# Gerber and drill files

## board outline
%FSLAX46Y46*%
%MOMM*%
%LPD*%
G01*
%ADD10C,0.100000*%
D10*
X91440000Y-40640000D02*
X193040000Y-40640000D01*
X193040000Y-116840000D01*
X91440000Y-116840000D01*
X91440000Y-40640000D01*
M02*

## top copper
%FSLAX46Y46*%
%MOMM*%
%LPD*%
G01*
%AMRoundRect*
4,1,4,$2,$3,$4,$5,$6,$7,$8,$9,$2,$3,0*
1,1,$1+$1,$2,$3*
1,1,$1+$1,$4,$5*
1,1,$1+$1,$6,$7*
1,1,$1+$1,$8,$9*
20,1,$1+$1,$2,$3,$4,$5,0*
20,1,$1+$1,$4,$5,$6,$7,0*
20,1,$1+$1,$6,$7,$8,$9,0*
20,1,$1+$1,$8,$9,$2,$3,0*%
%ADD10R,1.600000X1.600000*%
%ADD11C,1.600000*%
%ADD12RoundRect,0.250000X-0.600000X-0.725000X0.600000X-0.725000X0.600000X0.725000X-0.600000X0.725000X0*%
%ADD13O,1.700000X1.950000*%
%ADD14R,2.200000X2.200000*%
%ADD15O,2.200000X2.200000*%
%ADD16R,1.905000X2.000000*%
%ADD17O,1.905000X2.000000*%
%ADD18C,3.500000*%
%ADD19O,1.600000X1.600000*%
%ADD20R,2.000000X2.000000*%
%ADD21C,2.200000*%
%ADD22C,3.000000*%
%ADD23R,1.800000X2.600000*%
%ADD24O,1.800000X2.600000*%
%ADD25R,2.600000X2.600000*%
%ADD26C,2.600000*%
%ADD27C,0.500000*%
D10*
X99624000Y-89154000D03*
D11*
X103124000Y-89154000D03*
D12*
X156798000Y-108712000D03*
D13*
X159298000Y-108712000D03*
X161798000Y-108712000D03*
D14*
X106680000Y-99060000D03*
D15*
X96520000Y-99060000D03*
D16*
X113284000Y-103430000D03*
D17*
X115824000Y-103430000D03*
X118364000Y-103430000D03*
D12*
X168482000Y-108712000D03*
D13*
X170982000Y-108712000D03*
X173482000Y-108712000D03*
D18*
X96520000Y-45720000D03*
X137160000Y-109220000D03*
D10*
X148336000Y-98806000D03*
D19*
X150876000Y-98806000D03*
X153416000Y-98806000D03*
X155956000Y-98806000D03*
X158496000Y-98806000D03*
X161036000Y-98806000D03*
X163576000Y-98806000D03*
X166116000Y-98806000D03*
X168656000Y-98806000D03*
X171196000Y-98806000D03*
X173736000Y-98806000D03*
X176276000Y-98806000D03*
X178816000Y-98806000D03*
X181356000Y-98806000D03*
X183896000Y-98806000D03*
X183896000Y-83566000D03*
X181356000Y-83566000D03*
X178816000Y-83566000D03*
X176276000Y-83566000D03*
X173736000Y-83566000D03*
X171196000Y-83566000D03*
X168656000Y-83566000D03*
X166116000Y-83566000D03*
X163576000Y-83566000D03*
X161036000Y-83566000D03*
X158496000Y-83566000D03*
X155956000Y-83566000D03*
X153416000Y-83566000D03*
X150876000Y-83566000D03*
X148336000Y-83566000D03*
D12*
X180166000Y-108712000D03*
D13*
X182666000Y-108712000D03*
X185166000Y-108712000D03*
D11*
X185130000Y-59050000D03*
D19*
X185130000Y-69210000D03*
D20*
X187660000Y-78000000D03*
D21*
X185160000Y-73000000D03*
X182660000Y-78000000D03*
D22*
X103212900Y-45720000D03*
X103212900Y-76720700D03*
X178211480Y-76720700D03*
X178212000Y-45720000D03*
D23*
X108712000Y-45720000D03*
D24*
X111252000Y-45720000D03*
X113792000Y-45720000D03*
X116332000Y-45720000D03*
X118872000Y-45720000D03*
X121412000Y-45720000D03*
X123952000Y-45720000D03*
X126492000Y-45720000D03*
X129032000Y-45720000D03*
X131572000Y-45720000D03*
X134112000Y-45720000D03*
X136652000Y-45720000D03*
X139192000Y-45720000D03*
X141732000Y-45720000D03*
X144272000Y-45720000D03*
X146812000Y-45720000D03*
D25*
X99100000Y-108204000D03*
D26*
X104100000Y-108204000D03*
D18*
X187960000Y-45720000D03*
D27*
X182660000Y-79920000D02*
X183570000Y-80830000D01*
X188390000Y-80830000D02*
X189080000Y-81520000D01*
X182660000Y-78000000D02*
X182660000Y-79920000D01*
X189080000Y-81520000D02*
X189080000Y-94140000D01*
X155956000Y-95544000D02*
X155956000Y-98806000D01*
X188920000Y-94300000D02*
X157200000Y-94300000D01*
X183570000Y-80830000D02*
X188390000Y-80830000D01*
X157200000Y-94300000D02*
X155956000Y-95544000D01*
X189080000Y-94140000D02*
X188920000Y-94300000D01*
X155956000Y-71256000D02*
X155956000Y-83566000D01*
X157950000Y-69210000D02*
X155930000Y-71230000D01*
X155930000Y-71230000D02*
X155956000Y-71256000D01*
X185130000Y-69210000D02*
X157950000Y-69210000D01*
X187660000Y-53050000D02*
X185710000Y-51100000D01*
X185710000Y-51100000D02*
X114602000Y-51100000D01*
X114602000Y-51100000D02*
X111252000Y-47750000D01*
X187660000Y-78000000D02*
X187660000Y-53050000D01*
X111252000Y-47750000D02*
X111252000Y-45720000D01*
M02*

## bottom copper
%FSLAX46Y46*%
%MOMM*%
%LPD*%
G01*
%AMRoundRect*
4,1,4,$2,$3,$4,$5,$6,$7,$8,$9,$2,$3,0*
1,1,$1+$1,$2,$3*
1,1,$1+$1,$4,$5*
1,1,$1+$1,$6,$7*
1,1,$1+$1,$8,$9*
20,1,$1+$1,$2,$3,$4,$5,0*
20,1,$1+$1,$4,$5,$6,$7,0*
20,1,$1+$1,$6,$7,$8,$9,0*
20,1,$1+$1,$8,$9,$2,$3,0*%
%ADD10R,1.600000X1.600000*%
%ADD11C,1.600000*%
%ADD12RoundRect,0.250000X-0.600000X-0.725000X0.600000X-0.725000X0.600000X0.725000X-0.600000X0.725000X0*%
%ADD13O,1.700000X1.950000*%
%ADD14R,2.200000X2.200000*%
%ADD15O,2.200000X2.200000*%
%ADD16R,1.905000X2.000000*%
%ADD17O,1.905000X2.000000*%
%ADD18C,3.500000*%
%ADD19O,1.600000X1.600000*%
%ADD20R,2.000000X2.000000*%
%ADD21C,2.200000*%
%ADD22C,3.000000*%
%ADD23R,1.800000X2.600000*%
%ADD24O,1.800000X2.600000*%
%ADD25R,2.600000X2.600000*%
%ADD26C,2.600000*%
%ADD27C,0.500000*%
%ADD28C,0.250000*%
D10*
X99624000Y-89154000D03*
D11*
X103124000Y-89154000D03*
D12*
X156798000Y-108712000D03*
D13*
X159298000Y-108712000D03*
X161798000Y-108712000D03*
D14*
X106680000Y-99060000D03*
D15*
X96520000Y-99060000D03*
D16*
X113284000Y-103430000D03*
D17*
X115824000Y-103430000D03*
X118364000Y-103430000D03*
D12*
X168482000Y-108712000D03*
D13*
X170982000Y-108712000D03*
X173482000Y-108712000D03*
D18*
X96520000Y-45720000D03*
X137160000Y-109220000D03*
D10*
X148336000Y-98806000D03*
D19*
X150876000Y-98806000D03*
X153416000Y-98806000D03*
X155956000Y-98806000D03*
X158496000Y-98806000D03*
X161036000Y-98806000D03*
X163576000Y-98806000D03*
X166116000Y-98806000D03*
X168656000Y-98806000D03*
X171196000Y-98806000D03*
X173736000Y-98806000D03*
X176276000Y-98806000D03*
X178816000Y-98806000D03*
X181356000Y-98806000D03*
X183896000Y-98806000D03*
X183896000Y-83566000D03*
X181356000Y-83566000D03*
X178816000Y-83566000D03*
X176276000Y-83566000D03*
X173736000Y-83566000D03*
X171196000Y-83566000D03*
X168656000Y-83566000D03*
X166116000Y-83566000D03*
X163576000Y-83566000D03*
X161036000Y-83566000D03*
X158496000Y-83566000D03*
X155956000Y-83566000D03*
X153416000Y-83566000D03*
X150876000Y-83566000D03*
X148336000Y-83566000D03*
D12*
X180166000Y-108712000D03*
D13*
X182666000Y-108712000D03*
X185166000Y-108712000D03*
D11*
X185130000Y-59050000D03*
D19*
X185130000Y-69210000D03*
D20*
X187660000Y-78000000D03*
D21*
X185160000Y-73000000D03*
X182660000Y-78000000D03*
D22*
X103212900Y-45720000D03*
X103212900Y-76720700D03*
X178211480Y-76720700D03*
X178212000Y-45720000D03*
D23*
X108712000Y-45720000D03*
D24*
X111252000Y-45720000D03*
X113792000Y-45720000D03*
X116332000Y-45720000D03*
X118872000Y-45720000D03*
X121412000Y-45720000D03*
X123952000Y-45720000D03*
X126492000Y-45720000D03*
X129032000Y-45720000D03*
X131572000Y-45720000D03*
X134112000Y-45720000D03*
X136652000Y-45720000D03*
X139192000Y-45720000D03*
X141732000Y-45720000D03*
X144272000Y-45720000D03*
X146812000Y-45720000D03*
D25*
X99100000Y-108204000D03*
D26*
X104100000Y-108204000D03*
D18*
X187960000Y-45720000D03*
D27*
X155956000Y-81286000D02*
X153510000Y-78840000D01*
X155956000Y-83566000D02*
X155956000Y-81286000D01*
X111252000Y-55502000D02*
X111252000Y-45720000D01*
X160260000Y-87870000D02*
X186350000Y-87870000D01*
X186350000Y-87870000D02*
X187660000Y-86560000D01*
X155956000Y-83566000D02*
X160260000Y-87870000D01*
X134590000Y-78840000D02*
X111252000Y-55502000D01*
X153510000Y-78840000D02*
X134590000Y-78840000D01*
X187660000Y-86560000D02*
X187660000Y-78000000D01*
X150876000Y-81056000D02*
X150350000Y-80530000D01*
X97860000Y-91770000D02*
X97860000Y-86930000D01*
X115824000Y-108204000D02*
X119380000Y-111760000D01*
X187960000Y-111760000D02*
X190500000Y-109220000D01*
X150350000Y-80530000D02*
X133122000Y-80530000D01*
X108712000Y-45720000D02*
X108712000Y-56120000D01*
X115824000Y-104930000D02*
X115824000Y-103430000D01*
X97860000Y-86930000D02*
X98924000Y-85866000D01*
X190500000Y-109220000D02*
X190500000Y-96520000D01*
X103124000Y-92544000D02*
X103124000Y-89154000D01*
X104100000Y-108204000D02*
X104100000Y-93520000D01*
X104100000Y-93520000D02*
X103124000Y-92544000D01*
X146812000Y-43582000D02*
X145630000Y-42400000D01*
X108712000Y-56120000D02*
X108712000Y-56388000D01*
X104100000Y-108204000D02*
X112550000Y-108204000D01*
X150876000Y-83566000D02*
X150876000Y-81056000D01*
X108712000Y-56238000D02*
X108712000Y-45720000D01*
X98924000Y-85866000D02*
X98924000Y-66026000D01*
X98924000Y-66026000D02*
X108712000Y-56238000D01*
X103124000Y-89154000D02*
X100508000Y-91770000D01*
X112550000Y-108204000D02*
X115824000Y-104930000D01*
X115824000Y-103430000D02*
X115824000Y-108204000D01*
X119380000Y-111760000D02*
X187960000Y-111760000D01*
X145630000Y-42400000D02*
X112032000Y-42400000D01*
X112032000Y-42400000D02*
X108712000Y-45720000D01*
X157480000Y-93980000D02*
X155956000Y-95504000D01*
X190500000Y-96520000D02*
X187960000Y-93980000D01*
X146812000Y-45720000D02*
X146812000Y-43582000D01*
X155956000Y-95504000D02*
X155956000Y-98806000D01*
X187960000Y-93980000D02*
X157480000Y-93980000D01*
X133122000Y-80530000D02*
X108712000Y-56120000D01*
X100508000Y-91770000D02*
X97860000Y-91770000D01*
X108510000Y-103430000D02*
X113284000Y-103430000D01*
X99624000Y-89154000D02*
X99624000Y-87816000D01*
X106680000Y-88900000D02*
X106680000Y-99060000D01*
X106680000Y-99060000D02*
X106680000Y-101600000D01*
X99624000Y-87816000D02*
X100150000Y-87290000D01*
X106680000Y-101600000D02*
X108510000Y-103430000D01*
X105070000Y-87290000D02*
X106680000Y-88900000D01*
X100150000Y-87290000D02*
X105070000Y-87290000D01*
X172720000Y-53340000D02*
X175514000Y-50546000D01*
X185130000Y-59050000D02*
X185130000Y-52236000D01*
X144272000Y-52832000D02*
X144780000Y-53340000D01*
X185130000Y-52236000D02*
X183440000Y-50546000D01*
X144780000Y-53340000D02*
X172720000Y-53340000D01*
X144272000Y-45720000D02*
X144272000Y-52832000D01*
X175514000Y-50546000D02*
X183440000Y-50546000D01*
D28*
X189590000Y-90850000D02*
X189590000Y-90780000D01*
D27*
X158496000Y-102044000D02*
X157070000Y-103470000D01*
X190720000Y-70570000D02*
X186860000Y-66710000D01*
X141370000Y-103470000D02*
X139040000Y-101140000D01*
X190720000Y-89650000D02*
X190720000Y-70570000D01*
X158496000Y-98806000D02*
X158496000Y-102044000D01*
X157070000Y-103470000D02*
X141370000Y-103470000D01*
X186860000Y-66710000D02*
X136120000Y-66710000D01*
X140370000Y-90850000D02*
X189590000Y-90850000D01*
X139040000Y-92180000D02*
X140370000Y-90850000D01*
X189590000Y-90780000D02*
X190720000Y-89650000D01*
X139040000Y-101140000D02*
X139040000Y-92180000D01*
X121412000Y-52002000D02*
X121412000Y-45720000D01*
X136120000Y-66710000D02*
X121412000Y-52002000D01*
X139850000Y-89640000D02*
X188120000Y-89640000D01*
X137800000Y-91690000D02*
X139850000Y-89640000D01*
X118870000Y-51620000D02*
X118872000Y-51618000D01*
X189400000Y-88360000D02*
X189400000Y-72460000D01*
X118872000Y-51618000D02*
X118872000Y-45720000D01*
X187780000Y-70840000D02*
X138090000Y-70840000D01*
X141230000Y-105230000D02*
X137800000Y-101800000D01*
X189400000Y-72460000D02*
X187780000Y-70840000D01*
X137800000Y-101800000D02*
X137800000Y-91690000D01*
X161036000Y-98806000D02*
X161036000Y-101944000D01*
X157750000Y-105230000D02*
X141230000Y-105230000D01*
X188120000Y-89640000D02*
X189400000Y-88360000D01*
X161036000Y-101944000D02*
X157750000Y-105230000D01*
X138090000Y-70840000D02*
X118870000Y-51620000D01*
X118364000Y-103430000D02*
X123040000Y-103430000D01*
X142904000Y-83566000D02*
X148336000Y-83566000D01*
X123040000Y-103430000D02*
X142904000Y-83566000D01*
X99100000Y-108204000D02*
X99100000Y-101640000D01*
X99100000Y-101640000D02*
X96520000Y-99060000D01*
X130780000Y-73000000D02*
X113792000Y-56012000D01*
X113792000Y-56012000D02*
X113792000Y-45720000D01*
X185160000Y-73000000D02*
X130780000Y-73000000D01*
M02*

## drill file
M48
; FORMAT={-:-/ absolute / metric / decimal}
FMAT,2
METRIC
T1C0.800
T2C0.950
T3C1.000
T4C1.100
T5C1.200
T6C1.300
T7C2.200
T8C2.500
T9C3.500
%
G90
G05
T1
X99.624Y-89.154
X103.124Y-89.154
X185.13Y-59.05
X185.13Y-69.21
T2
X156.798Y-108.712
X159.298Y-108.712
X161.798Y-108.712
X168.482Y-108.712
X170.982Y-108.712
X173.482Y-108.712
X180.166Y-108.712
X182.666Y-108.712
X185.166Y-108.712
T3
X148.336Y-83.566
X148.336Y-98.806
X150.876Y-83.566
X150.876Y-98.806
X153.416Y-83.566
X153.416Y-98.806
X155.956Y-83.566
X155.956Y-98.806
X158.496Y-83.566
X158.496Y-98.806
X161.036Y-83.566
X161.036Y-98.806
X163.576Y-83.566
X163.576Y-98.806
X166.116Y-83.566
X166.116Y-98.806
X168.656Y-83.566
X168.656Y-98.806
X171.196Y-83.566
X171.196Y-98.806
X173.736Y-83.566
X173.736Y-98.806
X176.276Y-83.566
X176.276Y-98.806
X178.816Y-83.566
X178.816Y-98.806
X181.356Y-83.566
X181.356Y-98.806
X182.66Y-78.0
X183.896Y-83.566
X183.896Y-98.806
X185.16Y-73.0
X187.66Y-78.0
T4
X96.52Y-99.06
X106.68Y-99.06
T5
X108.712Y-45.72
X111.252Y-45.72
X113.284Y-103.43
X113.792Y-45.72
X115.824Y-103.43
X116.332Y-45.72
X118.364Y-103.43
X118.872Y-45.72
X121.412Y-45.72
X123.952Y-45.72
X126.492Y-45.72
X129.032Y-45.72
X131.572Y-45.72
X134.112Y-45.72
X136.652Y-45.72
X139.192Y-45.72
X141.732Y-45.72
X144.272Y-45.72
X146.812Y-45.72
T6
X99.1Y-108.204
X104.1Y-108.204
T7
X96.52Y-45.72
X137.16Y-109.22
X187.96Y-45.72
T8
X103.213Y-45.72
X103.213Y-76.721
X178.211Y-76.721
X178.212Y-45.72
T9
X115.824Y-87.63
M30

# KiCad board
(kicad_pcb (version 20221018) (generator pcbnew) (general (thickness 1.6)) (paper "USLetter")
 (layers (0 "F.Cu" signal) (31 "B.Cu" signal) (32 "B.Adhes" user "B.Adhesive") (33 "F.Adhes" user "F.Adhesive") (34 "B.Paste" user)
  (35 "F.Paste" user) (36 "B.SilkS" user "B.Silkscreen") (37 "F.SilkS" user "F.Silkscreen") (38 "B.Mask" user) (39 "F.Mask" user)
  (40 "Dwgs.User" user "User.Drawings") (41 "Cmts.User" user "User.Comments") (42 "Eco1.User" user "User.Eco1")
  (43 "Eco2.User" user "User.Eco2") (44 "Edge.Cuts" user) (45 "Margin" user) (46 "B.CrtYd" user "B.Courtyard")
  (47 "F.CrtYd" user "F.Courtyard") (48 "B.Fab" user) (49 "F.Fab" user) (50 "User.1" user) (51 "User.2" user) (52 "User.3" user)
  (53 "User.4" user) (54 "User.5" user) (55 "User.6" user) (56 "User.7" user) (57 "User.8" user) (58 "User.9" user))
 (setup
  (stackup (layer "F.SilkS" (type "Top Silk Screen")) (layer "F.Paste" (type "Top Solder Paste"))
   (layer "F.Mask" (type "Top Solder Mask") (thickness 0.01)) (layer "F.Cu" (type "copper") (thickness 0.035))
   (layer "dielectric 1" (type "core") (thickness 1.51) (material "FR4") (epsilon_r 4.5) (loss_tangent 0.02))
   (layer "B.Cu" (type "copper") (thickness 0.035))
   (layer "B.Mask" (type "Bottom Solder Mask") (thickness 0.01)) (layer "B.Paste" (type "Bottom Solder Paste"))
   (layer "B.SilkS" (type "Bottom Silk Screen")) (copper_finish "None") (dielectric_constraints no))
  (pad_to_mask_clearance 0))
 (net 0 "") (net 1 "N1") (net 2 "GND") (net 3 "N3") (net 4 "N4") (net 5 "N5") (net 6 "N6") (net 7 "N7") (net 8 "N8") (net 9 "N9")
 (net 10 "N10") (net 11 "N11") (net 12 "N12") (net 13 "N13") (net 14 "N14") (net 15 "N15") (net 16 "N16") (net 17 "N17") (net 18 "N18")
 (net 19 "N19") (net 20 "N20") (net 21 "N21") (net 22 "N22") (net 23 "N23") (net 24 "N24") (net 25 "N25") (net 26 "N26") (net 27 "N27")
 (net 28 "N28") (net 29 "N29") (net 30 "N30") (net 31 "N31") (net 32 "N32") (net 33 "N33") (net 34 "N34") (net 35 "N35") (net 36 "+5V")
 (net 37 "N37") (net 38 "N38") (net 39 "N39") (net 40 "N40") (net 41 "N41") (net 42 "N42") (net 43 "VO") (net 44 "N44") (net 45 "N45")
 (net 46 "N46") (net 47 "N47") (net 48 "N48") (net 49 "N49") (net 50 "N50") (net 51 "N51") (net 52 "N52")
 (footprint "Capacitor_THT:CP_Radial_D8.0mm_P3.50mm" (layer "F.Cu") (at 99.624 89.154)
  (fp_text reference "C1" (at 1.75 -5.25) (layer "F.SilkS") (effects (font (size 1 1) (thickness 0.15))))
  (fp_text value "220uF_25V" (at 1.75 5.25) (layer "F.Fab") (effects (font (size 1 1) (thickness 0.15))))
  (pad "1" thru_hole rect (at 0 0) (size 1.6 1.6) (drill 0.8) (layers "*.Cu" "*.Mask") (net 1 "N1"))
  (pad "2" thru_hole circle (at 3.5 0) (size 1.6 1.6) (drill 0.8) (layers "*.Cu" "*.Mask") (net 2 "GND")))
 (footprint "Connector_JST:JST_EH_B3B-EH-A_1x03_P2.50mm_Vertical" (layer "F.Cu") (at 156.798 108.712)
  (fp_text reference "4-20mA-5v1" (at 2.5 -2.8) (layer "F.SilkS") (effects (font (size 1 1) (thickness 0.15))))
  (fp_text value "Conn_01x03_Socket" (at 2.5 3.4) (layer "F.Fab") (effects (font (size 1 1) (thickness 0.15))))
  (pad "1" thru_hole roundrect (at 0 0) (size 1.7 1.95) (drill 0.95) (layers "*.Cu" "*.Mask") (roundrect_rratio 0.147059) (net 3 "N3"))
  (pad "2" thru_hole oval (at 2.5 0) (size 1.7 1.95) (drill 0.95) (layers "*.Cu" "*.Mask") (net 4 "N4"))
  (pad "3" thru_hole oval (at 5 0) (size 1.7 1.95) (drill 0.95) (layers "*.Cu" "*.Mask") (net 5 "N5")))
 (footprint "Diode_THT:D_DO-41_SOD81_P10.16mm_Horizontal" (layer "F.Cu") (at 106.68 99.06 180)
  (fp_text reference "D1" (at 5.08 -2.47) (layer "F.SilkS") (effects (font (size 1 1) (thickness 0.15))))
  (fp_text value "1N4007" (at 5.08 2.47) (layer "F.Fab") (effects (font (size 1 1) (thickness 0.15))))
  (pad "1" thru_hole rect (at 0 0 180) (size 2.2 2.2) (drill 1.1) (layers "*.Cu" "*.Mask") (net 1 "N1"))
  (pad "2" thru_hole oval (at 10.16 0 180) (size 2.2 2.2) (drill 1.1) (layers "*.Cu" "*.Mask") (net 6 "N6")))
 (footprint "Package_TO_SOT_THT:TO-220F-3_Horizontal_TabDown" (layer "F.Cu") (at 113.284 103.43)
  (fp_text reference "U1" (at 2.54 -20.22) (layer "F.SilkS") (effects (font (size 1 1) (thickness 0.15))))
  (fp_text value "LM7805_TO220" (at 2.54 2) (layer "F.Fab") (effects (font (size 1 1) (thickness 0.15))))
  (pad "" np_thru_hole oval (at 2.54 -15.8) (size 3.5 3.5) (drill 3.5) (layers "*.Cu" "*.Mask"))
  (pad "1" thru_hole rect (at 0 0) (size 1.905 2) (drill 1.2) (layers "*.Cu" "*.Mask") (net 1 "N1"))
  (pad "2" thru_hole oval (at 2.54 0) (size 1.905 2) (drill 1.2) (layers "*.Cu" "*.Mask") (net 2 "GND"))
  (pad "3" thru_hole oval (at 5.08 0) (size 1.905 2) (drill 1.2) (layers "*.Cu" "*.Mask") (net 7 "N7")))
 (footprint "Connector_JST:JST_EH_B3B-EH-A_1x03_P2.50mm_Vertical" (layer "F.Cu") (at 168.482 108.712)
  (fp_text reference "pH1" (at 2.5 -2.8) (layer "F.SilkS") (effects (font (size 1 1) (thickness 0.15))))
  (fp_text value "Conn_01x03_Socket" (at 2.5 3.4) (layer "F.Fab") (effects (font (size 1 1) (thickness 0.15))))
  (pad "1" thru_hole roundrect (at 0 0) (size 1.7 1.95) (drill 0.95) (layers "*.Cu" "*.Mask") (roundrect_rratio 0.147059) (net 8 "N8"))
  (pad "2" thru_hole oval (at 2.5 0) (size 1.7 1.95) (drill 0.95) (layers "*.Cu" "*.Mask") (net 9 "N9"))
  (pad "3" thru_hole oval (at 5 0) (size 1.7 1.95) (drill 0.95) (layers "*.Cu" "*.Mask") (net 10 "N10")))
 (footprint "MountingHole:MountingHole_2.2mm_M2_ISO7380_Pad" (layer "F.Cu") (at 96.52 45.72)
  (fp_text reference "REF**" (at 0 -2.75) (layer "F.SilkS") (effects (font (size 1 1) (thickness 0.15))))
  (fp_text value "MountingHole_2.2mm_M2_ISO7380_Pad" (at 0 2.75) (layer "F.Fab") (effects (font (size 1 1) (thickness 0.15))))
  (pad "1" thru_hole circle (at 0 0) (size 3.5 3.5) (drill 2.2) (layers "*.Cu" "*.Mask")))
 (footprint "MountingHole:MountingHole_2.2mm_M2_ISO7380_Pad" (layer "F.Cu") (at 137.16 109.22)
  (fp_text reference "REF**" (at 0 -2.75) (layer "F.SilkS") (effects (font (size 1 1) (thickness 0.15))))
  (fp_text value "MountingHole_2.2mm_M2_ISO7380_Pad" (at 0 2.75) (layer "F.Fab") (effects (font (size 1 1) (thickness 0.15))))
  (pad "1" thru_hole circle (at 0 0) (size 3.5 3.5) (drill 2.2) (layers "*.Cu" "*.Mask")))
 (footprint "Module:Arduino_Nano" (layer "F.Cu") (at 148.336 98.806 90)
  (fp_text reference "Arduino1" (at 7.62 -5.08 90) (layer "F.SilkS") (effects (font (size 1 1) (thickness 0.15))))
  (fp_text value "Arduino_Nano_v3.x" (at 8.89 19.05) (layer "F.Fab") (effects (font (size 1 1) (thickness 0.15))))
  (pad "1" thru_hole rect (at 0 0 90) (size 1.6 1.6) (drill 1) (layers "*.Cu" "*.Mask") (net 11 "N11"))
  (pad "2" thru_hole oval (at 0 2.54 90) (size 1.6 1.6) (drill 1) (layers "*.Cu" "*.Mask") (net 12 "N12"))
  (pad "3" thru_hole oval (at 0 5.08 90) (size 1.6 1.6) (drill 1) (layers "*.Cu" "*.Mask") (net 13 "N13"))
  (pad "4" thru_hole oval (at 0 7.62 90) (size 1.6 1.6) (drill 1) (layers "*.Cu" "*.Mask") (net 2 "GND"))
  (pad "5" thru_hole oval (at 0 10.16 90) (size 1.6 1.6) (drill 1) (layers "*.Cu" "*.Mask") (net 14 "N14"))
  (pad "6" thru_hole oval (at 0 12.7 90) (size 1.6 1.6) (drill 1) (layers "*.Cu" "*.Mask") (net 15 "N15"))
  (pad "7" thru_hole oval (at 0 15.24 90) (size 1.6 1.6) (drill 1) (layers "*.Cu" "*.Mask") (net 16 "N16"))
  (pad "8" thru_hole oval (at 0 17.78 90) (size 1.6 1.6) (drill 1) (layers "*.Cu" "*.Mask") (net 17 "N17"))
  (pad "9" thru_hole oval (at 0 20.32 90) (size 1.6 1.6) (drill 1) (layers "*.Cu" "*.Mask") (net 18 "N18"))
  (pad "10" thru_hole oval (at 0 22.86 90) (size 1.6 1.6) (drill 1) (layers "*.Cu" "*.Mask") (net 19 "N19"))
  (pad "11" thru_hole oval (at 0 25.4 90) (size 1.6 1.6) (drill 1) (layers "*.Cu" "*.Mask") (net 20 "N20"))
  (pad "12" thru_hole oval (at 0 27.94 90) (size 1.6 1.6) (drill 1) (layers "*.Cu" "*.Mask") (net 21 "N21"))
  (pad "13" thru_hole oval (at 0 30.48 90) (size 1.6 1.6) (drill 1) (layers "*.Cu" "*.Mask") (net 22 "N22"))
  (pad "14" thru_hole oval (at 0 33.02 90) (size 1.6 1.6) (drill 1) (layers "*.Cu" "*.Mask") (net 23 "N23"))
  (pad "15" thru_hole oval (at 0 35.56 90) (size 1.6 1.6) (drill 1) (layers "*.Cu" "*.Mask") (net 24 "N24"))
  (pad "16" thru_hole oval (at 15.24 35.56 90) (size 1.6 1.6) (drill 1) (layers "*.Cu" "*.Mask") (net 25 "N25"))
  (pad "17" thru_hole oval (at 15.24 33.02 90) (size 1.6 1.6) (drill 1) (layers "*.Cu" "*.Mask") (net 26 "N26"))
  (pad "18" thru_hole oval (at 15.24 30.48 90) (size 1.6 1.6) (drill 1) (layers "*.Cu" "*.Mask") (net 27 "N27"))
  (pad "19" thru_hole oval (at 15.24 27.94 90) (size 1.6 1.6) (drill 1) (layers "*.Cu" "*.Mask") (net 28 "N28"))
  (pad "20" thru_hole oval (at 15.24 25.4 90) (size 1.6 1.6) (drill 1) (layers "*.Cu" "*.Mask") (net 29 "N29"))
  (pad "21" thru_hole oval (at 15.24 22.86 90) (size 1.6 1.6) (drill 1) (layers "*.Cu" "*.Mask") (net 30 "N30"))
  (pad "22" thru_hole oval (at 15.24 20.32 90) (size 1.6 1.6) (drill 1) (layers "*.Cu" "*.Mask") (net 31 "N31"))
  (pad "23" thru_hole oval (at 15.24 17.78 90) (size 1.6 1.6) (drill 1) (layers "*.Cu" "*.Mask") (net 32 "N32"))
  (pad "24" thru_hole oval (at 15.24 15.24 90) (size 1.6 1.6) (drill 1) (layers "*.Cu" "*.Mask") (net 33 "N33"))
  (pad "25" thru_hole oval (at 15.24 12.7 90) (size 1.6 1.6) (drill 1) (layers "*.Cu" "*.Mask") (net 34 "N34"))
  (pad "26" thru_hole oval (at 15.24 10.16 90) (size 1.6 1.6) (drill 1) (layers "*.Cu" "*.Mask") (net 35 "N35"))
  (pad "27" thru_hole oval (at 15.24 7.62 90) (size 1.6 1.6) (drill 1) (layers "*.Cu" "*.Mask") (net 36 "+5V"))
  (pad "28" thru_hole oval (at 15.24 5.08 90) (size 1.6 1.6) (drill 1) (layers "*.Cu" "*.Mask") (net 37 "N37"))
  (pad "29" thru_hole oval (at 15.24 2.54 90) (size 1.6 1.6) (drill 1) (layers "*.Cu" "*.Mask") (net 2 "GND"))
  (pad "30" thru_hole oval (at 15.24 0 90) (size 1.6 1.6) (drill 1) (layers "*.Cu" "*.Mask") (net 7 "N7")))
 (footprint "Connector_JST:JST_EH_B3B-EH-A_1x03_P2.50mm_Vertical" (layer "F.Cu") (at 180.166 108.712)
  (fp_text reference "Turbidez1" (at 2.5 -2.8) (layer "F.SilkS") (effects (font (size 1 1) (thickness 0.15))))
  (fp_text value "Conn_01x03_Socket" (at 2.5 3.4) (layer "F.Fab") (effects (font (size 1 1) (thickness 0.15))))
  (pad "1" thru_hole roundrect (at 0 0) (size 1.7 1.95) (drill 0.95) (layers "*.Cu" "*.Mask") (roundrect_rratio 0.147059) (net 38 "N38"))
  (pad "2" thru_hole oval (at 2.5 0) (size 1.7 1.95) (drill 0.95) (layers "*.Cu" "*.Mask") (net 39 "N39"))
  (pad "3" thru_hole oval (at 5 0) (size 1.7 1.95) (drill 0.95) (layers "*.Cu" "*.Mask") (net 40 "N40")))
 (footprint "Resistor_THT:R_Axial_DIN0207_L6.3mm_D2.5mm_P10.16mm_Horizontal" (layer "F.Cu") (at 185.13 59.05 -90)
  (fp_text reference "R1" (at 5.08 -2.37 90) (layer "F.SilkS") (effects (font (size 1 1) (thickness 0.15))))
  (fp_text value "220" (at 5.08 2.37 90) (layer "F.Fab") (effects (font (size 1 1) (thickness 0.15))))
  (pad "1" thru_hole circle (at 0 0 270) (size 1.6 1.6) (drill 0.8) (layers "*.Cu" "*.Mask") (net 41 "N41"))
  (pad "2" thru_hole oval (at 10.16 0 270) (size 1.6 1.6) (drill 0.8) (layers "*.Cu" "*.Mask") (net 36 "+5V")))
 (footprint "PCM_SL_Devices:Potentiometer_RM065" (layer "F.Cu") (at 185.13 75.97 180)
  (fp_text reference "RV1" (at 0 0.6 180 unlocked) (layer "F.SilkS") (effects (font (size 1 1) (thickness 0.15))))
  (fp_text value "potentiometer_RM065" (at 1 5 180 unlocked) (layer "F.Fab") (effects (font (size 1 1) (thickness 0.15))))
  (pad "1" thru_hole rect (at -2.53 -2.03 180) (size 2 2) (drill 1) (layers "*.Cu" "*.Mask") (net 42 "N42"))
  (pad "2" thru_hole circle (at -0.03 2.97 180) (size 2.2 2.2) (drill 1) (layers "*.Cu" "*.Mask") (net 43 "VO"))
  (pad "3" thru_hole circle (at 2.47 -2.03 180) (size 2.2 2.2) (drill 1) (layers "*.Cu" "*.Mask") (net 2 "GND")))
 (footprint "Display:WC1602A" (layer "F.Cu") (at 108.712 45.72)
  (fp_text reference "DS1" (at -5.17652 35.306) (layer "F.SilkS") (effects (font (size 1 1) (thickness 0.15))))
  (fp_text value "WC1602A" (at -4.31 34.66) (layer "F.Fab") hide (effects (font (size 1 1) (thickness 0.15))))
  (pad "" thru_hole circle (at -5.4991 0) (size 3 3) (drill 2.5) (layers "*.Cu" "*.Mask"))
  (pad "" thru_hole circle (at -5.4991 31.0007) (size 3 3) (drill 2.5) (layers "*.Cu" "*.Mask"))
  (pad "" thru_hole circle (at 69.49948 31.0007) (size 3 3) (drill 2.5) (layers "*.Cu" "*.Mask"))
  (pad "" thru_hole circle (at 69.5 0) (size 3 3) (drill 2.5) (layers "*.Cu" "*.Mask"))
  (pad "1" thru_hole rect (at 0 0) (size 1.8 2.6) (drill 1.2) (layers "*.Cu" "*.Mask") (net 2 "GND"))
  (pad "2" thru_hole oval (at 2.54 0) (size 1.8 2.6) (drill 1.2) (layers "*.Cu" "*.Mask") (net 42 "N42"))
  (pad "3" thru_hole oval (at 5.08 0) (size 1.8 2.6) (drill 1.2) (layers "*.Cu" "*.Mask") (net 43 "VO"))
  (pad "4" thru_hole oval (at 7.62 0) (size 1.8 2.6) (drill 1.2) (layers "*.Cu" "*.Mask") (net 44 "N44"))
  (pad "5" thru_hole oval (at 10.16 0) (size 1.8 2.6) (drill 1.2) (layers "*.Cu" "*.Mask") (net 15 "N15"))
  (pad "6" thru_hole oval (at 12.7 0) (size 1.8 2.6) (drill 1.2) (layers "*.Cu" "*.Mask") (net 14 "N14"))
  (pad "7" thru_hole oval (at 15.24 0) (size 1.8 2.6) (drill 1.2) (layers "*.Cu" "*.Mask") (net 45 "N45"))
  (pad "8" thru_hole oval (at 17.78 0) (size 1.8 2.6) (drill 1.2) (layers "*.Cu" "*.Mask") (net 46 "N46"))
  (pad "9" thru_hole oval (at 20.32 0) (size 1.8 2.6) (drill 1.2) (layers "*.Cu" "*.Mask") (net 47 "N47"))
  (pad "10" thru_hole oval (at 22.86 0) (size 1.8 2.6) (drill 1.2) (layers "*.Cu" "*.Mask") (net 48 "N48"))
  (pad "11" thru_hole oval (at 25.4 0) (size 1.8 2.6) (drill 1.2) (layers "*.Cu" "*.Mask") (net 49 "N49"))
  (pad "12" thru_hole oval (at 27.94 0) (size 1.8 2.6) (drill 1.2) (layers "*.Cu" "*.Mask") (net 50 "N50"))
  (pad "13" thru_hole oval (at 30.48 0) (size 1.8 2.6) (drill 1.2) (layers "*.Cu" "*.Mask") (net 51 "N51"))
  (pad "14" thru_hole oval (at 33.02 0) (size 1.8 2.6) (drill 1.2) (layers "*.Cu" "*.Mask") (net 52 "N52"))
  (pad "15" thru_hole oval (at 35.56 0) (size 1.8 2.6) (drill 1.2) (layers "*.Cu" "*.Mask") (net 41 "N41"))
  (pad "16" thru_hole oval (at 38.1 0) (size 1.8 2.6) (drill 1.2) (layers "*.Cu" "*.Mask") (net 2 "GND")))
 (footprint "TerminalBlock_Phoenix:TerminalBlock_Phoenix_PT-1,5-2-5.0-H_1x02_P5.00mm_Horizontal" (layer "F.Cu") (at 99.1 108.204)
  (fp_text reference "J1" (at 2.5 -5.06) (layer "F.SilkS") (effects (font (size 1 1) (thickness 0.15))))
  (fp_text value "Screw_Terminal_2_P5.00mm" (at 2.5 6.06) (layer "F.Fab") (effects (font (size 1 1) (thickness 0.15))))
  (pad "1" thru_hole rect (at 0 0) (size 2.6 2.6) (drill 1.3) (layers "*.Cu" "*.Mask") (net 6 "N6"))
  (pad "2" thru_hole circle (at 5 0) (size 2.6 2.6) (drill 1.3) (layers "*.Cu" "*.Mask") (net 2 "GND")))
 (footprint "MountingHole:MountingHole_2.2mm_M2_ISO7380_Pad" (layer "F.Cu") (at 187.96 45.72)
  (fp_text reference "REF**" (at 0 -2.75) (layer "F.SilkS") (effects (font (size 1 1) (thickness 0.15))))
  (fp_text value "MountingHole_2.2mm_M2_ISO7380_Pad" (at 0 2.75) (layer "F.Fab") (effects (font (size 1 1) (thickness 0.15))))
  (pad "1" thru_hole circle (at 0 0) (size 3.5 3.5) (drill 2.2) (layers "*.Cu" "*.Mask")))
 (gr_rect (start 105.31 137.08) (end 105.31 137.08) (stroke (width 0.1) (type default)) (fill none) (layer "Edge.Cuts"))
 (gr_rect (start 91.44 40.64) (end 193.04 116.84) (stroke (width 0.1) (type default)) (fill none) (layer "Edge.Cuts"))
 (segment (start 155.956 81.286) (end 153.51 78.84) (width 0.5) (layer "B.Cu") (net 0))
 (segment (start 155.956 83.566) (end 155.956 81.286) (width 0.5) (layer "B.Cu") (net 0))
 (segment (start 111.252 55.502) (end 111.252 45.72) (width 0.5) (layer "B.Cu") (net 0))
 (segment (start 160.26 87.87) (end 186.35 87.87) (width 0.5) (layer "B.Cu") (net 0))
 (segment (start 186.35 87.87) (end 187.66 86.56) (width 0.5) (layer "B.Cu") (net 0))
 (segment (start 155.956 83.566) (end 160.26 87.87) (width 0.5) (layer "B.Cu") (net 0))
 (segment (start 134.59 78.84) (end 111.252 55.502) (width 0.5) (layer "B.Cu") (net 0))
 (segment (start 153.51 78.84) (end 134.59 78.84) (width 0.5) (layer "B.Cu") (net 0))
 (segment (start 187.66 86.56) (end 187.66 78) (width 0.5) (layer "B.Cu") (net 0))
 (segment (start 182.66 79.92) (end 183.57 80.83) (width 0.5) (layer "F.Cu") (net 2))
 (segment (start 188.39 80.83) (end 189.08 81.52) (width 0.5) (layer "F.Cu") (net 2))
 (segment (start 182.66 78) (end 182.66 79.92) (width 0.5) (layer "F.Cu") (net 2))
 (segment (start 189.08 81.52) (end 189.08 94.14) (width 0.5) (layer "F.Cu") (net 2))
 (segment (start 155.956 95.544) (end 155.956 98.806) (width 0.5) (layer "F.Cu") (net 2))
 (segment (start 188.92 94.3) (end 157.2 94.3) (width 0.5) (layer "F.Cu") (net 2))
 (segment (start 183.57 80.83) (end 188.39 80.83) (width 0.5) (layer "F.Cu") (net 2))
 (segment (start 157.2 94.3) (end 155.956 95.544) (width 0.5) (layer "F.Cu") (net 2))
 (segment (start 189.08 94.14) (end 188.92 94.3) (width 0.5) (layer "F.Cu") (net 2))
 (segment (start 150.876 81.056) (end 150.35 80.53) (width 0.5) (layer "B.Cu") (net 2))
 (segment (start 97.86 91.77) (end 97.86 86.93) (width 0.5) (layer "B.Cu") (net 2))
 (segment (start 115.824 108.204) (end 119.38 111.76) (width 0.5) (layer "B.Cu") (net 2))
 (segment (start 187.96 111.76) (end 190.5 109.22) (width 0.5) (layer "B.Cu") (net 2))
 (segment (start 150.35 80.53) (end 133.122 80.53) (width 0.5) (layer "B.Cu") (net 2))
 (segment (start 108.712 45.72) (end 108.712 56.12) (width 0.5) (layer "B.Cu") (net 2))
 (segment (start 115.824 104.93) (end 115.824 103.43) (width 0.5) (layer "B.Cu") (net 2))
 (segment (start 97.86 86.93) (end 98.924 85.866) (width 0.5) (layer "B.Cu") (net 2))
 (segment (start 190.5 109.22) (end 190.5 96.52) (width 0.5) (layer "B.Cu") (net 2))
 (segment (start 103.124 92.544) (end 103.124 89.154) (width 0.5) (layer "B.Cu") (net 2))
 (segment (start 104.1 108.204) (end 104.1 93.52) (width 0.5) (layer "B.Cu") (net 2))
 (segment (start 104.1 93.52) (end 103.124 92.544) (width 0.5) (layer "B.Cu") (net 2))
 (segment (start 146.812 43.582) (end 145.63 42.4) (width 0.5) (layer "B.Cu") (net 2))
 (segment (start 108.712 56.12) (end 108.712 56.388) (width 0.5) (layer "B.Cu") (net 2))
 (segment (start 104.1 108.204) (end 112.55 108.204) (width 0.5) (layer "B.Cu") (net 2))
 (segment (start 150.876 83.566) (end 150.876 81.056) (width 0.5) (layer "B.Cu") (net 2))
 (segment (start 108.712 56.238) (end 108.712 45.72) (width 0.5) (layer "B.Cu") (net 2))
 (segment (start 98.924 85.866) (end 98.924 66.026) (width 0.5) (layer "B.Cu") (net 2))
 (segment (start 98.924 66.026) (end 108.712 56.238) (width 0.5) (layer "B.Cu") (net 2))
 (segment (start 103.124 89.154) (end 100.508 91.77) (width 0.5) (layer "B.Cu") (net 2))
 (segment (start 112.55 108.204) (end 115.824 104.93) (width 0.5) (layer "B.Cu") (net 2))
 (segment (start 115.824 103.43) (end 115.824 108.204) (width 0.5) (layer "B.Cu") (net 2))
 (segment (start 119.38 111.76) (end 187.96 111.76) (width 0.5) (layer "B.Cu") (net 2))
 (segment (start 145.63 42.4) (end 112.032 42.4) (width 0.5) (layer "B.Cu") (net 2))
 (segment (start 112.032 42.4) (end 108.712 45.72) (width 0.5) (layer "B.Cu") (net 2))
 (segment (start 157.48 93.98) (end 155.956 95.504) (width 0.5) (layer "B.Cu") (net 2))
 (segment (start 190.5 96.52) (end 187.96 93.98) (width 0.5) (layer "B.Cu") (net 2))
 (segment (start 146.812 45.72) (end 146.812 43.582) (width 0.5) (layer "B.Cu") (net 2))
 (segment (start 155.956 95.504) (end 155.956 98.806) (width 0.5) (layer "B.Cu") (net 2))
 (segment (start 187.96 93.98) (end 157.48 93.98) (width 0.5) (layer "B.Cu") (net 2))
 (segment (start 133.122 80.53) (end 108.712 56.12) (width 0.5) (layer "B.Cu") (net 2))
 (segment (start 100.508 91.77) (end 97.86 91.77) (width 0.5) (layer "B.Cu") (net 2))
 (segment (start 108.51 103.43) (end 113.284 103.43) (width 0.5) (layer "B.Cu") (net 1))
 (segment (start 99.624 89.154) (end 99.624 87.816) (width 0.5) (layer "B.Cu") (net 1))
 (segment (start 106.68 88.9) (end 106.68 99.06) (width 0.5) (layer "B.Cu") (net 1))
 (segment (start 106.68 99.06) (end 106.68 101.6) (width 0.5) (layer "B.Cu") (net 1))
 (segment (start 99.624 87.816) (end 100.15 87.29) (width 0.5) (layer "B.Cu") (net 1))
 (segment (start 106.68 101.6) (end 108.51 103.43) (width 0.5) (layer "B.Cu") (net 1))
 (segment (start 105.07 87.29) (end 106.68 88.9) (width 0.5) (layer "B.Cu") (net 1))
 (segment (start 100.15 87.29) (end 105.07 87.29) (width 0.5) (layer "B.Cu") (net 1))
 (segment (start 155.956 71.256) (end 155.956 83.566) (width 0.5) (layer "F.Cu") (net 36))
 (segment (start 157.95 69.21) (end 155.93 71.23) (width 0.5) (layer "F.Cu") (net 36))
 (segment (start 155.93 71.23) (end 155.956 71.256) (width 0.5) (layer "F.Cu") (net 36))
 (segment (start 185.13 69.21) (end 157.95 69.21) (width 0.5) (layer "F.Cu") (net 36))
 (segment (start 172.72 53.34) (end 175.514 50.546) (width 0.5) (layer "B.Cu") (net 41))
 (segment (start 185.13 59.05) (end 185.13 52.236) (width 0.5) (layer "B.Cu") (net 41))
 (segment (start 144.272 52.832) (end 144.78 53.34) (width 0.5) (layer "B.Cu") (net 41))
 (segment (start 185.13 52.236) (end 183.44 50.546) (width 0.5) (layer "B.Cu") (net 41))
 (segment (start 144.78 53.34) (end 172.72 53.34) (width 0.5) (layer "B.Cu") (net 41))
 (segment (start 144.272 45.72) (end 144.272 52.832) (width 0.5) (layer "B.Cu") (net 41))
 (segment (start 175.514 50.546) (end 183.44 50.546) (width 0.5) (layer "B.Cu") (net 41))
 (segment (start 187.66 53.05) (end 185.71 51.1) (width 0.5) (layer "F.Cu") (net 42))
 (segment (start 185.71 51.1) (end 114.602 51.1) (width 0.5) (layer "F.Cu") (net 42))
 (segment (start 114.602 51.1) (end 111.252 47.75) (width 0.5) (layer "F.Cu") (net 42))
 (segment (start 187.66 78) (end 187.66 53.05) (width 0.5) (layer "F.Cu") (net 42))
 (segment (start 111.252 47.75) (end 111.252 45.72) (width 0.5) (layer "F.Cu") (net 42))
 (segment (start 189.59 90.85) (end 189.59 90.78) (width 0.25) (layer "B.Cu") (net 14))
 (segment (start 158.496 102.044) (end 157.07 103.47) (width 0.5) (layer "B.Cu") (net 14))
 (segment (start 190.72 70.57) (end 186.86 66.71) (width 0.5) (layer "B.Cu") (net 14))
 (segment (start 141.37 103.47) (end 139.04 101.14) (width 0.5) (layer "B.Cu") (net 14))
 (segment (start 190.72 89.65) (end 190.72 70.57) (width 0.5) (layer "B.Cu") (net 14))
 (segment (start 158.496 98.806) (end 158.496 102.044) (width 0.5) (layer "B.Cu") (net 14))
 (segment (start 157.07 103.47) (end 141.37 103.47) (width 0.5) (layer "B.Cu") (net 14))
 (segment (start 186.86 66.71) (end 136.12 66.71) (width 0.5) (layer "B.Cu") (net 14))
 (segment (start 140.37 90.85) (end 189.59 90.85) (width 0.5) (layer "B.Cu") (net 14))
 (segment (start 139.04 92.18) (end 140.37 90.85) (width 0.5) (layer "B.Cu") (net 14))
 (segment (start 189.59 90.78) (end 190.72 89.65) (width 0.5) (layer "B.Cu") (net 14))
 (segment (start 139.04 101.14) (end 139.04 92.18) (width 0.5) (layer "B.Cu") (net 14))
 (segment (start 121.412 52.002) (end 121.412 45.72) (width 0.5) (layer "B.Cu") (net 14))
 (segment (start 136.12 66.71) (end 121.412 52.002) (width 0.5) (layer "B.Cu") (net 14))
 (segment (start 139.85 89.64) (end 188.12 89.64) (width 0.5) (layer "B.Cu") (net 15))
 (segment (start 137.8 91.69) (end 139.85 89.64) (width 0.5) (layer "B.Cu") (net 15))
 (segment (start 118.87 51.62) (end 118.872 51.618) (width 0.5) (layer "B.Cu") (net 15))
 (segment (start 189.4 88.36) (end 189.4 72.46) (width 0.5) (layer "B.Cu") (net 15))
 (segment (start 118.872 51.618) (end 118.872 45.72) (width 0.5) (layer "B.Cu") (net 15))
 (segment (start 187.78 70.84) (end 138.09 70.84) (width 0.5) (layer "B.Cu") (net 15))
 (segment (start 141.23 105.23) (end 137.8 101.8) (width 0.5) (layer "B.Cu") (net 15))
 (segment (start 189.4 72.46) (end 187.78 70.84) (width 0.5) (layer "B.Cu") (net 15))
 (segment (start 137.8 101.8) (end 137.8 91.69) (width 0.5) (layer "B.Cu") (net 15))
 (segment (start 161.036 98.806) (end 161.036 101.944) (width 0.5) (layer "B.Cu") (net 15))
 (segment (start 157.75 105.23) (end 141.23 105.23) (width 0.5) (layer "B.Cu") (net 15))
 (segment (start 188.12 89.64) (end 189.4 88.36) (width 0.5) (layer "B.Cu") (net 15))
 (segment (start 161.036 101.944) (end 157.75 105.23) (width 0.5) (layer "B.Cu") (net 15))
 (segment (start 138.09 70.84) (end 118.87 51.62) (width 0.5) (layer "B.Cu") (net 15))
 (segment (start 118.364 103.43) (end 123.04 103.43) (width 0.5) (layer "B.Cu") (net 7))
 (segment (start 142.904 83.566) (end 148.336 83.566) (width 0.5) (layer "B.Cu") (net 7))
 (segment (start 123.04 103.43) (end 142.904 83.566) (width 0.5) (layer "B.Cu") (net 7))
 (segment (start 99.1 108.204) (end 99.1 101.64) (width 0.5) (layer "B.Cu") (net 6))
 (segment (start 99.1 101.64) (end 96.52 99.06) (width 0.5) (layer "B.Cu") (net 6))
 (segment (start 130.78 73) (end 113.792 56.012) (width 0.5) (layer "B.Cu") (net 43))
 (segment (start 113.792 56.012) (end 113.792 45.72) (width 0.5) (layer "B.Cu") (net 43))
 (segment (start 185.16 73) (end 130.78 73) (width 0.5) (layer "B.Cu") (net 43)))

